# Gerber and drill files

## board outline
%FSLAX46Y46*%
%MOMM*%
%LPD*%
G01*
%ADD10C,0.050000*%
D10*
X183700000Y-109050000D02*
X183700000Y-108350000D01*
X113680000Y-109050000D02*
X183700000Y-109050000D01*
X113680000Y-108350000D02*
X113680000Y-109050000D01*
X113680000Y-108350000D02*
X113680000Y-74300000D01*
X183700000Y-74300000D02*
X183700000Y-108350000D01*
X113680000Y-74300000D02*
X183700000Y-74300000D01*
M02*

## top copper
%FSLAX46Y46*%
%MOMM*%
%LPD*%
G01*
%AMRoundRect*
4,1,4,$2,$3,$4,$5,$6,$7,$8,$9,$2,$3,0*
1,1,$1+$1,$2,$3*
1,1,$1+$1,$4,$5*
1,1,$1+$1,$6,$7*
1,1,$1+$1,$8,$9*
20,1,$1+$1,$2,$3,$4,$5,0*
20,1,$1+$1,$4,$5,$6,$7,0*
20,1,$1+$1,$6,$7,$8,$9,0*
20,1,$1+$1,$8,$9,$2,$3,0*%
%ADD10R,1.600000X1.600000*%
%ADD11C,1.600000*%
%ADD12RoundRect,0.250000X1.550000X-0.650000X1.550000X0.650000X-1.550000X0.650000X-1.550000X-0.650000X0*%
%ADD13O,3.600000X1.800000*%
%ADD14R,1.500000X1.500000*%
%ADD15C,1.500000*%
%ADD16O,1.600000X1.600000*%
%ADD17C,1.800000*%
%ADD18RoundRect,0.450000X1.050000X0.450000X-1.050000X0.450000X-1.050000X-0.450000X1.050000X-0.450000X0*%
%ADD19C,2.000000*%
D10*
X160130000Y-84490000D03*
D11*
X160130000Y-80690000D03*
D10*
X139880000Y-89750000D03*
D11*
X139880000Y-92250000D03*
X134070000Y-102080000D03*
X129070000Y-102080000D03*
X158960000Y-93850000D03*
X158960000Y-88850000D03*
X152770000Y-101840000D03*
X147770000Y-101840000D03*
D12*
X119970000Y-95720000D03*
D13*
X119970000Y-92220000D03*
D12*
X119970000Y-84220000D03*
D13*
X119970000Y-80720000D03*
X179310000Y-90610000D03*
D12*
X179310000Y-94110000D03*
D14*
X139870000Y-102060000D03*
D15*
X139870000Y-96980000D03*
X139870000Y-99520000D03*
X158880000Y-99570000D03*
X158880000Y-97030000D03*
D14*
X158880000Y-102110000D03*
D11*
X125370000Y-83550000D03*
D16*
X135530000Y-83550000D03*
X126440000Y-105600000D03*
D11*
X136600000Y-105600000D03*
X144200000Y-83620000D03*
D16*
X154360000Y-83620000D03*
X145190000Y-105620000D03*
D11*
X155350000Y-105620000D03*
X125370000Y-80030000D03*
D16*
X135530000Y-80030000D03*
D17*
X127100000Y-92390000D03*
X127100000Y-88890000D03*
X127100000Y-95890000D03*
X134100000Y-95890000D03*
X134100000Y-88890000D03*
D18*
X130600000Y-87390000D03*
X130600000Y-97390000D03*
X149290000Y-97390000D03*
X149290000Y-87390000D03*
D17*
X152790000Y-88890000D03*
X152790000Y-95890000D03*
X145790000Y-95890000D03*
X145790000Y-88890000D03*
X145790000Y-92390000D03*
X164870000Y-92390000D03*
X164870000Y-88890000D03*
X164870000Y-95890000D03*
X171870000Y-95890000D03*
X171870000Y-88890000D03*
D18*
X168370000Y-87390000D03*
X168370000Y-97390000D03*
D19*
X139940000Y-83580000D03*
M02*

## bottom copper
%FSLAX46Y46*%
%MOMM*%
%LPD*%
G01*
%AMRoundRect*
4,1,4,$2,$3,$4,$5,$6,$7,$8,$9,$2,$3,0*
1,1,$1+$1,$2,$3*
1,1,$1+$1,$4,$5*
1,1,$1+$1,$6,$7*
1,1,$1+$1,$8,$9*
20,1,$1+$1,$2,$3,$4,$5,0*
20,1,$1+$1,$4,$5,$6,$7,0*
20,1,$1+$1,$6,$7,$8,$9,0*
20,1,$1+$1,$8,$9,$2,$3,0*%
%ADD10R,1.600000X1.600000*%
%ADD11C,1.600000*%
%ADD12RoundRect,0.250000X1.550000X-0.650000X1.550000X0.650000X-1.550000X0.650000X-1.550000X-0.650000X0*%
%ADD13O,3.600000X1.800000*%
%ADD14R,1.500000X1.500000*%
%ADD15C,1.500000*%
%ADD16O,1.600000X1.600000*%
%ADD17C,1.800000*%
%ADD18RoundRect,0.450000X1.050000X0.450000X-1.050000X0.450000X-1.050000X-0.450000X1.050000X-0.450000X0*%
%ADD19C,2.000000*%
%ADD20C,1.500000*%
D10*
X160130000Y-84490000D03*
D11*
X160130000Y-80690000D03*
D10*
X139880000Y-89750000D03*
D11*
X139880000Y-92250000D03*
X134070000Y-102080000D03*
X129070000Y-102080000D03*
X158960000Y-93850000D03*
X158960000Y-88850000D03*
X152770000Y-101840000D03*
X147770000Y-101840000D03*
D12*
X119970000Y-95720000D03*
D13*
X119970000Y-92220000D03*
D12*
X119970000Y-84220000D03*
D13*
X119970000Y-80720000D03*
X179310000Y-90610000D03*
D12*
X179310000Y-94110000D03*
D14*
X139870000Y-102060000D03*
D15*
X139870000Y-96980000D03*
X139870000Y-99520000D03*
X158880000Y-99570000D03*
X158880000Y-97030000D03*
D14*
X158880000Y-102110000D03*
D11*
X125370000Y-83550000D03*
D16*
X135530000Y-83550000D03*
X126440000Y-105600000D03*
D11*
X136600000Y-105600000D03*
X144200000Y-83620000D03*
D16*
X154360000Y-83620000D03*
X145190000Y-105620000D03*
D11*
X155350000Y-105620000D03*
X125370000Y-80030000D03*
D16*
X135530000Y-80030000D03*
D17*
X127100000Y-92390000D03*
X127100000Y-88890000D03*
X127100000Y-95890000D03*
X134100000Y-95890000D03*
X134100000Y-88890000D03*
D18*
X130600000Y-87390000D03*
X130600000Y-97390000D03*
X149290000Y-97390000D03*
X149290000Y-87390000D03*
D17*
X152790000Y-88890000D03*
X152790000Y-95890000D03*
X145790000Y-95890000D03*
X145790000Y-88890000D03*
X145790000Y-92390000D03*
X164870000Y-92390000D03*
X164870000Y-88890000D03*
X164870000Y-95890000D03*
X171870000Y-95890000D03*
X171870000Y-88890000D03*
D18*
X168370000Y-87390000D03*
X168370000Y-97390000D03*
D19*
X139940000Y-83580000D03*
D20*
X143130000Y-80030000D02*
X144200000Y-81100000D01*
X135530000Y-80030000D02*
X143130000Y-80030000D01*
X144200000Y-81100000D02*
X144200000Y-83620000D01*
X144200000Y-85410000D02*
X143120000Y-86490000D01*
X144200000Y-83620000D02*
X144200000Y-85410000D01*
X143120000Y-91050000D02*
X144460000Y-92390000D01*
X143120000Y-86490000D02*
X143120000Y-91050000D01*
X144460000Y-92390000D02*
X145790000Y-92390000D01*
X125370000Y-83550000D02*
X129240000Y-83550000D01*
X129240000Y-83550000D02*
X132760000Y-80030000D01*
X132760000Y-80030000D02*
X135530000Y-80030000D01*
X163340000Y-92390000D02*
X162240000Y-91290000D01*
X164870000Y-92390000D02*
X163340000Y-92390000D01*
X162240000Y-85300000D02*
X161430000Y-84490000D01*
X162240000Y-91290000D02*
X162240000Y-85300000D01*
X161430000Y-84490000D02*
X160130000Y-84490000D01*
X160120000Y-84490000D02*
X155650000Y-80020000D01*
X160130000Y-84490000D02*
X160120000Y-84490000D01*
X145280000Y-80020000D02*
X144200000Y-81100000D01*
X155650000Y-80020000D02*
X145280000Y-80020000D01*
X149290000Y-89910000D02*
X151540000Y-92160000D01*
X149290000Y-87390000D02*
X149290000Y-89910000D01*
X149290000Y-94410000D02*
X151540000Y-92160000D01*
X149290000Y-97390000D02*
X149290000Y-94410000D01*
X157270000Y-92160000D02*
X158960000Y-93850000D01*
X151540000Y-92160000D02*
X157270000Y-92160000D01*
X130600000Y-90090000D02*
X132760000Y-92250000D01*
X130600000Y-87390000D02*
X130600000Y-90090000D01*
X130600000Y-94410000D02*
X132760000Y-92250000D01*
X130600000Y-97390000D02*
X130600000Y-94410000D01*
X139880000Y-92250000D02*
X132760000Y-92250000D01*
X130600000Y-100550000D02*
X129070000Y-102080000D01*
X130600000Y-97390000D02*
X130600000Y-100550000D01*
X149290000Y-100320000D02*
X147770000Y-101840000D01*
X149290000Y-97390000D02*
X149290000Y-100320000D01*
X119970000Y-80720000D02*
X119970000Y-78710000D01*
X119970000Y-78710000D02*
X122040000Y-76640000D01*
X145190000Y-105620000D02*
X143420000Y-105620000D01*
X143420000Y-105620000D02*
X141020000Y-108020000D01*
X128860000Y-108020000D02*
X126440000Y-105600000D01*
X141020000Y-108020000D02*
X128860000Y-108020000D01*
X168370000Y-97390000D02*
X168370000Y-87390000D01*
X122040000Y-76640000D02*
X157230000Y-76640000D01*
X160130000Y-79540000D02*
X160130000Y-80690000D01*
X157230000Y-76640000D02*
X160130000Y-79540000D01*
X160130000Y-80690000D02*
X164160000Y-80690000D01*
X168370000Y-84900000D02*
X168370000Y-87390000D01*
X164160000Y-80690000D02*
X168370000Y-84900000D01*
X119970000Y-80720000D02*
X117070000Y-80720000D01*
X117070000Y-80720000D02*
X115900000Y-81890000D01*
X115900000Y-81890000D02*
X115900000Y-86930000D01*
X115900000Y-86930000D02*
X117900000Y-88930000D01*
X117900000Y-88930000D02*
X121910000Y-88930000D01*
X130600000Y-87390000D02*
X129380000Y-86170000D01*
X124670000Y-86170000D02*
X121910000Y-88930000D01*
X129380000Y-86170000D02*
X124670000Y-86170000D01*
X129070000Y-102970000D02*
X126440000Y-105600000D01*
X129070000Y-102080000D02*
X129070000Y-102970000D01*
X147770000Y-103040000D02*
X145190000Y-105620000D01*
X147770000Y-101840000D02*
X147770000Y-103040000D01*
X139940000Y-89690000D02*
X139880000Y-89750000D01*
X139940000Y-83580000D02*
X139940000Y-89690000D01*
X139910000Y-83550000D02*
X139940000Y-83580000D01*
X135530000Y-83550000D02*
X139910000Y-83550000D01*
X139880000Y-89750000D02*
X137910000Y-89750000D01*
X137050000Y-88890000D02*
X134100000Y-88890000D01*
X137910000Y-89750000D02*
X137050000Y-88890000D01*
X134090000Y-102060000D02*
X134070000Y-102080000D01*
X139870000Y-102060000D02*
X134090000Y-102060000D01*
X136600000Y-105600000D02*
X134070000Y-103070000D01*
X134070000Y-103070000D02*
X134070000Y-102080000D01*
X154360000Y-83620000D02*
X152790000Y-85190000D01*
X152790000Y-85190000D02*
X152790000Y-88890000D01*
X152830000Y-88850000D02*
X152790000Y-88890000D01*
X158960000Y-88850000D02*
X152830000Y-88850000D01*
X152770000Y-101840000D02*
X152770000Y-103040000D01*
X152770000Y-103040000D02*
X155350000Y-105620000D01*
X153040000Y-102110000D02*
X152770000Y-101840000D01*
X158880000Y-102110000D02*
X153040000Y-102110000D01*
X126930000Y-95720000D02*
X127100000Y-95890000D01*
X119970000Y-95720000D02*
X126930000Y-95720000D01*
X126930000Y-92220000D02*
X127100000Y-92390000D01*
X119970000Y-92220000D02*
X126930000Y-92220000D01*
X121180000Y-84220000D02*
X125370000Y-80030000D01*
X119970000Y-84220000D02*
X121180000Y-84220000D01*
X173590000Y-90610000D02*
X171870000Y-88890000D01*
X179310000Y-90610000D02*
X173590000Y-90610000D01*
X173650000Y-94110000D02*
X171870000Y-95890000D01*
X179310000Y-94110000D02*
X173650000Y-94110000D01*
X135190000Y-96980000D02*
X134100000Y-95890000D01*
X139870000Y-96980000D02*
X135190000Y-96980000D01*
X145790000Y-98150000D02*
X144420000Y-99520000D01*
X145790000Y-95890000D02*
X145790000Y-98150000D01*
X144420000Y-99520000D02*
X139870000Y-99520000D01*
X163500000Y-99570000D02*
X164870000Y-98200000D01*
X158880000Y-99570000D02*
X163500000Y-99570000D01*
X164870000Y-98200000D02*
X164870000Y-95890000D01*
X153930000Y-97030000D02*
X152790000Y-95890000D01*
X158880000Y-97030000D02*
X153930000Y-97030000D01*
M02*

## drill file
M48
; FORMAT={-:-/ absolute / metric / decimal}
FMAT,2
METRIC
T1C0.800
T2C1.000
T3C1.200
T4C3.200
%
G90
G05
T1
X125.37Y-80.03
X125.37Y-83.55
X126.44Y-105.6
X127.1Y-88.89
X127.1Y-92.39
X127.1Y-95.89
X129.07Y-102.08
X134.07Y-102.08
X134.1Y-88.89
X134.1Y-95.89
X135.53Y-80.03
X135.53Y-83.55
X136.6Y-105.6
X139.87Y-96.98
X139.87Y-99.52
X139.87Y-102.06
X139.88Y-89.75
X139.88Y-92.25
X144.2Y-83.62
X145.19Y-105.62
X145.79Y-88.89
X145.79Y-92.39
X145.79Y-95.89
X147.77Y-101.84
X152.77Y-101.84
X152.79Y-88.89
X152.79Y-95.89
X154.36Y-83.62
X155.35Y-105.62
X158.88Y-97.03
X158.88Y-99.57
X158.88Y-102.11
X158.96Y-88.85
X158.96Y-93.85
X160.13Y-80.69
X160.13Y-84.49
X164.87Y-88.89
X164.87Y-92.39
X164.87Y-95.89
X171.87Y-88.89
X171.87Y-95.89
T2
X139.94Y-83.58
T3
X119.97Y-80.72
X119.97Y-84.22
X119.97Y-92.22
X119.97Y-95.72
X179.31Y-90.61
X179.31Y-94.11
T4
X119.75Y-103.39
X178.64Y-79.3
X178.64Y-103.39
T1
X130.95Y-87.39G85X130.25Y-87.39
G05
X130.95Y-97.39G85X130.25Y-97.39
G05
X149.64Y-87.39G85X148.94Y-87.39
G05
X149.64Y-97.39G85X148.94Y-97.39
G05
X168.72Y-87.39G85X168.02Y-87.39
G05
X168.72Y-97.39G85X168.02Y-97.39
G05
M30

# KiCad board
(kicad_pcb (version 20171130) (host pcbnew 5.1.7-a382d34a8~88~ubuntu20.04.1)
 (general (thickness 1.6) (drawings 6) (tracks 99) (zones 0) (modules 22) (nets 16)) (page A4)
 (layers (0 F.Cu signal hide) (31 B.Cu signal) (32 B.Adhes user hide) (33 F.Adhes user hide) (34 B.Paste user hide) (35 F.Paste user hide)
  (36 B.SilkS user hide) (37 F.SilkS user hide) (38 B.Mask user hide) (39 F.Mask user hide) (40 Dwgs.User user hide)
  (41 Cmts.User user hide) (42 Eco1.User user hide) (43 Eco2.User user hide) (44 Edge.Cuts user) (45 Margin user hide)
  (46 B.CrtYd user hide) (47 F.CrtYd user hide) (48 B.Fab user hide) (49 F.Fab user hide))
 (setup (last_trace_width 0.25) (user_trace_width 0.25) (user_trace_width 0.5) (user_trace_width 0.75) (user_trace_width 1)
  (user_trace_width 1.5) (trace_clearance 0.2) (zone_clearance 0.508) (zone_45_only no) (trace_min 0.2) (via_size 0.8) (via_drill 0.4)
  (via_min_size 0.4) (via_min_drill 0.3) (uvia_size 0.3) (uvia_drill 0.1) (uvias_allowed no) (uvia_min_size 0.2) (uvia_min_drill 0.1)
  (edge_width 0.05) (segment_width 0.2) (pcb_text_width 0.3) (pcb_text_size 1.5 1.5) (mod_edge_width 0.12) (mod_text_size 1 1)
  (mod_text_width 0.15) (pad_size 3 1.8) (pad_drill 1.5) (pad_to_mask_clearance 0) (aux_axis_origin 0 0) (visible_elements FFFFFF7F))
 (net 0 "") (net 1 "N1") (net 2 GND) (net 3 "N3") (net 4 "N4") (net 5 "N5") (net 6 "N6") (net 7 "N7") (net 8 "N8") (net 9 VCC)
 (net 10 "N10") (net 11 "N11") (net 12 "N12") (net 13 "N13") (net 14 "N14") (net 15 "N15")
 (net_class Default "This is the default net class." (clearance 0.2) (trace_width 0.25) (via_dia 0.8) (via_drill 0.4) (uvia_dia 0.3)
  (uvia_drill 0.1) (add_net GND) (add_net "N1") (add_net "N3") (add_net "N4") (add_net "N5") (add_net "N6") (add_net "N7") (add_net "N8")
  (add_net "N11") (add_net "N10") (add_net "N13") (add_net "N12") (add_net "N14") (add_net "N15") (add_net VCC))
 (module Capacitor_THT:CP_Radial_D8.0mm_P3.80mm (layer F.Cu) (at 160.13 84.49 90)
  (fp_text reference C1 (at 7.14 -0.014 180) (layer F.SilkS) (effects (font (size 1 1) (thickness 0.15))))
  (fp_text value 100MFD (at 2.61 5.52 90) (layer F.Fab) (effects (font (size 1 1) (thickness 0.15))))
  (pad 1 thru_hole rect (at 0 0 90) (size 1.6 1.6) (drill 0.8) (layers *.Cu *.Mask) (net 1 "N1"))
  (pad 2 thru_hole circle (at 3.8 0 90) (size 1.6 1.6) (drill 0.8) (layers *.Cu *.Mask) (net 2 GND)))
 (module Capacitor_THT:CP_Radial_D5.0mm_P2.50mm (layer F.Cu) (at 139.88 89.75 270)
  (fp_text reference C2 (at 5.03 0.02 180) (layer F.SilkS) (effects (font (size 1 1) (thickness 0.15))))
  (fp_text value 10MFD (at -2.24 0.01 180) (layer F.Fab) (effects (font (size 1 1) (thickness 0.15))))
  (pad 1 thru_hole rect (at 0 0 270) (size 1.6 1.6) (drill 0.8) (layers *.Cu *.Mask) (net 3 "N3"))
  (pad 2 thru_hole circle (at 2.5 0 270) (size 1.6 1.6) (drill 0.8) (layers *.Cu *.Mask) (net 2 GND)))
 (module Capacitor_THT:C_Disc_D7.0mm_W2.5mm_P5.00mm (layer F.Cu) (at 134.07 102.08 180)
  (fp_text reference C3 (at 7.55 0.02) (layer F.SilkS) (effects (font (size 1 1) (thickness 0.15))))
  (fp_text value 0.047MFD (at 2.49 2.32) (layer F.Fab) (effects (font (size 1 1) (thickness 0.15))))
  (pad 1 thru_hole circle (at 0 0 180) (size 1.6 1.6) (drill 0.8) (layers *.Cu *.Mask) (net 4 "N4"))
  (pad 2 thru_hole circle (at 5 0 180) (size 1.6 1.6) (drill 0.8) (layers *.Cu *.Mask) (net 2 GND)))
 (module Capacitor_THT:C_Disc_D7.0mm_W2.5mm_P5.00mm (layer F.Cu) (at 158.96 88.85 270)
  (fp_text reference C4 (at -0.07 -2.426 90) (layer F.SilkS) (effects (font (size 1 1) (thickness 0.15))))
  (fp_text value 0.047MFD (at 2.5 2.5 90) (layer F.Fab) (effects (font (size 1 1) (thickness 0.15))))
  (pad 2 thru_hole circle (at 5 0 270) (size 1.6 1.6) (drill 0.8) (layers *.Cu *.Mask) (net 2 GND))
  (pad 1 thru_hole circle (at 0 0 270) (size 1.6 1.6) (drill 0.8) (layers *.Cu *.Mask) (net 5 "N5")))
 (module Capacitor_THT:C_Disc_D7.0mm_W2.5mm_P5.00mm (layer F.Cu) (at 152.77 101.84 180)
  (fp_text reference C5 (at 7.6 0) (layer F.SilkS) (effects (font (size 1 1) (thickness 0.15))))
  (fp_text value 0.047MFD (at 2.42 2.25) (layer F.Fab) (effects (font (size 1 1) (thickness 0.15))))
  (pad 1 thru_hole circle (at 0 0 180) (size 1.6 1.6) (drill 0.8) (layers *.Cu *.Mask) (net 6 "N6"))
  (pad 2 thru_hole circle (at 5 0 180) (size 1.6 1.6) (drill 0.8) (layers *.Cu *.Mask) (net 2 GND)))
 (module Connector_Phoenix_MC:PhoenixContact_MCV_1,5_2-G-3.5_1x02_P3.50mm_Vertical (layer F.Cu) (at 119.97 95.72 90)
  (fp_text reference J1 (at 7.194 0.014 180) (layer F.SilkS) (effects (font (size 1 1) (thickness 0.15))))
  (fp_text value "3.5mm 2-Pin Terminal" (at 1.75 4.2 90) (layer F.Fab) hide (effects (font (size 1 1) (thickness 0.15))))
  (pad 1 thru_hole roundrect (at 0 0 90) (size 1.8 3.6) (drill 1.2) (layers *.Cu *.Mask) (roundrect_rratio 0.138889) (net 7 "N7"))
  (pad 2 thru_hole oval (at 3.5 0 90) (size 1.8 3.6) (drill 1.2) (layers *.Cu *.Mask) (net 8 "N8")))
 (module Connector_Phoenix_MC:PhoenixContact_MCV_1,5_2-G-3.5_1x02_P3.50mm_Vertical (layer F.Cu) (at 119.97 84.22 90)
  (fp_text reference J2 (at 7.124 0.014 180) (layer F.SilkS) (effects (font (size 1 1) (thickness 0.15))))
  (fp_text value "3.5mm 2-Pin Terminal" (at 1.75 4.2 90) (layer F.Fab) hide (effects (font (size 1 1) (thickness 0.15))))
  (pad 1 thru_hole roundrect (at 0 0 90) (size 1.8 3.6) (drill 1.2) (layers *.Cu *.Mask) (roundrect_rratio 0.138889) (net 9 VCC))
  (pad 2 thru_hole oval (at 3.5 0 90) (size 1.8 3.6) (drill 1.2) (layers *.Cu *.Mask) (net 2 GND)))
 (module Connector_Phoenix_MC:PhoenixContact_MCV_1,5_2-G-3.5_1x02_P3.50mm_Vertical (layer F.Cu) (at 179.31 94.11 90)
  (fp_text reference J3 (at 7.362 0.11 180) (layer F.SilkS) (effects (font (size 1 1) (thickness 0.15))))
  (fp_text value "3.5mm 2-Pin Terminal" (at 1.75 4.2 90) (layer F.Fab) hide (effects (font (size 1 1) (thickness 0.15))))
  (pad 2 thru_hole oval (at 3.5 0 90) (size 1.8 3.6) (drill 1.2) (layers *.Cu *.Mask) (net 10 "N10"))
  (pad 1 thru_hole roundrect (at 0 0 90) (size 1.8 3.6) (drill 1.2) (layers *.Cu *.Mask) (roundrect_rratio 0.138889) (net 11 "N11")))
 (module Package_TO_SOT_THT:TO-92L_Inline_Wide (layer F.Cu) (at 139.87 102.06 90)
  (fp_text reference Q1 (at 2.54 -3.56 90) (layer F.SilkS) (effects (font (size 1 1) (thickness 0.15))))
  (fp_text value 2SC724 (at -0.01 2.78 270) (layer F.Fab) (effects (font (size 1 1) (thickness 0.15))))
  (pad 1 thru_hole rect (at 0 0 90) (size 1.5 1.5) (drill 0.8) (layers *.Cu *.Mask) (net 4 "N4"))
  (pad 3 thru_hole circle (at 5.08 0 90) (size 1.5 1.5) (drill 0.8) (layers *.Cu *.Mask) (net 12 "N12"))
  (pad 2 thru_hole circle (at 2.54 0 90) (size 1.5 1.5) (drill 0.8) (layers *.Cu *.Mask) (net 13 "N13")))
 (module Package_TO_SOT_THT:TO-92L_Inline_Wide (layer F.Cu) (at 158.88 102.11 90)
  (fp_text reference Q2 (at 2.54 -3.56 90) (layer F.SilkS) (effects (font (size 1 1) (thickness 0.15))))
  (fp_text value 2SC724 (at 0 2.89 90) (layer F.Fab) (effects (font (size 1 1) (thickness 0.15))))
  (pad 2 thru_hole circle (at 2.54 0 90) (size 1.5 1.5) (drill 0.8) (layers *.Cu *.Mask) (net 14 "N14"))
  (pad 3 thru_hole circle (at 5.08 0 90) (size 1.5 1.5) (drill 0.8) (layers *.Cu *.Mask) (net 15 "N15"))
  (pad 1 thru_hole rect (at 0 0 90) (size 1.5 1.5) (drill 0.8) (layers *.Cu *.Mask) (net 6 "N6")))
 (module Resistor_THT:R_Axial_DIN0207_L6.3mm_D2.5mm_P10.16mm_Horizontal (layer F.Cu) (at 125.37 83.55)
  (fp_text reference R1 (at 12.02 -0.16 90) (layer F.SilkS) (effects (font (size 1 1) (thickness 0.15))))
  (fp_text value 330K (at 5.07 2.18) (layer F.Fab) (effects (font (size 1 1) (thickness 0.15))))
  (pad 1 thru_hole circle (at 0 0) (size 1.6 1.6) (drill 0.8) (layers *.Cu *.Mask) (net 1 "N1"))
  (pad 2 thru_hole oval (at 10.16 0) (size 1.6 1.6) (drill 0.8) (layers *.Cu *.Mask) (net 3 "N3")))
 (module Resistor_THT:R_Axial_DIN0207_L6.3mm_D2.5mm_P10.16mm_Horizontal (layer F.Cu) (at 136.6 105.6 180)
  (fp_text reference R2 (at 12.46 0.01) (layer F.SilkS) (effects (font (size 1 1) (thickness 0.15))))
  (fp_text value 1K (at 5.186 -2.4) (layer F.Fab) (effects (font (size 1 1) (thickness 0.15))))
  (pad 2 thru_hole oval (at 10.16 0 180) (size 1.6 1.6) (drill 0.8) (layers *.Cu *.Mask) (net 2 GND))
  (pad 1 thru_hole circle (at 0 0 180) (size 1.6 1.6) (drill 0.8) (layers *.Cu *.Mask) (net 4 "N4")))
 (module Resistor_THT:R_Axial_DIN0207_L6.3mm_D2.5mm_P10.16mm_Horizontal (layer F.Cu) (at 144.2 83.62)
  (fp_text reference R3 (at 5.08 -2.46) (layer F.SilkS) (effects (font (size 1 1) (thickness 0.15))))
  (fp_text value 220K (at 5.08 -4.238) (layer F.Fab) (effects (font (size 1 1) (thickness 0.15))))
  (pad 1 thru_hole circle (at 0 0) (size 1.6 1.6) (drill 0.8) (layers *.Cu *.Mask) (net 1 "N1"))
  (pad 2 thru_hole oval (at 10.16 0) (size 1.6 1.6) (drill 0.8) (layers *.Cu *.Mask) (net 5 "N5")))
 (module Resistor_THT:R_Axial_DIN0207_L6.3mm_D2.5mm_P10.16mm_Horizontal (layer F.Cu) (at 155.35 105.62 180)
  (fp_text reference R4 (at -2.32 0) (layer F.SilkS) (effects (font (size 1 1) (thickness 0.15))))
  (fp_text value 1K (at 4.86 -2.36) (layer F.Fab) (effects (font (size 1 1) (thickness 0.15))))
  (pad 2 thru_hole oval (at 10.16 0 180) (size 1.6 1.6) (drill 0.8) (layers *.Cu *.Mask) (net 2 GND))
  (pad 1 thru_hole circle (at 0 0 180) (size 1.6 1.6) (drill 0.8) (layers *.Cu *.Mask) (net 6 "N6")))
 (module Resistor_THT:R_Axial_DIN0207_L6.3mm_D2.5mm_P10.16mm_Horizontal (layer F.Cu) (at 125.37 80.03)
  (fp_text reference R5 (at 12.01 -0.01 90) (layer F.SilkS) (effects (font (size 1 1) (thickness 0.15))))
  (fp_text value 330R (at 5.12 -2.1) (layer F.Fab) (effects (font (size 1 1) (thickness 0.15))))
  (pad 1 thru_hole circle (at 0 0) (size 1.6 1.6) (drill 0.8) (layers *.Cu *.Mask) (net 9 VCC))
  (pad 2 thru_hole oval (at 10.16 0) (size 1.6 1.6) (drill 0.8) (layers *.Cu *.Mask) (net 1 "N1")))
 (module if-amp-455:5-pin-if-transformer (layer F.Cu) (at 127.1 92.39 90)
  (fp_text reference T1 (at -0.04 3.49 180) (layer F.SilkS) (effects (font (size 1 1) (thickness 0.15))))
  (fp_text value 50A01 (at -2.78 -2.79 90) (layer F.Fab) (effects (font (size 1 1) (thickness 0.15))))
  (pad 2 thru_hole circle (at 0 0 90) (size 1.8 1.8) (drill 0.8) (layers *.Cu *.Mask) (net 8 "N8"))
  (pad 1 thru_hole circle (at 3.5 0 90) (size 1.8 1.8) (drill 0.8) (layers *.Cu *.Mask))
  (pad 3 thru_hole circle (at -3.5 0 90) (size 1.8 1.8) (drill 0.8) (layers *.Cu *.Mask) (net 7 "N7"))
  (pad 4 thru_hole circle (at -3.5 7 90) (size 1.8 1.8) (drill 0.8) (layers *.Cu *.Mask) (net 12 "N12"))
  (pad 5 thru_hole circle (at 3.5 7 90) (size 1.8 1.8) (drill 0.8) (layers *.Cu *.Mask) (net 3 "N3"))
  (pad 6 thru_hole roundrect (at 5 3.5 180) (size 3 1.8) (drill oval 1.5 0.8) (layers *.Cu *.Mask) (roundrect_rratio 0.25) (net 2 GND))
  (pad 6 thru_hole roundrect (at -5 3.5 180) (size 3 1.8) (drill oval 1.5 0.8) (layers *.Cu *.Mask) (roundrect_rratio 0.25) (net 2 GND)))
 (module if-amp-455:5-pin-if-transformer (layer F.Cu) (at 145.79 92.39 90)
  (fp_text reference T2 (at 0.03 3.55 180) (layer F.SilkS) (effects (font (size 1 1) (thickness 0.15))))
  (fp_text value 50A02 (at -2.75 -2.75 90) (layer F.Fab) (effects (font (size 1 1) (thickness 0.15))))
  (pad 6 thru_hole roundrect (at -5 3.5 180) (size 3 1.8) (drill oval 1.5 0.8) (layers *.Cu *.Mask) (roundrect_rratio 0.25) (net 2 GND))
  (pad 6 thru_hole roundrect (at 5 3.5 180) (size 3 1.8) (drill oval 1.5 0.8) (layers *.Cu *.Mask) (roundrect_rratio 0.25) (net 2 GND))
  (pad 5 thru_hole circle (at 3.5 7 90) (size 1.8 1.8) (drill 0.8) (layers *.Cu *.Mask) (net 5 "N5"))
  (pad 4 thru_hole circle (at -3.5 7 90) (size 1.8 1.8) (drill 0.8) (layers *.Cu *.Mask) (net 15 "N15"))
  (pad 3 thru_hole circle (at -3.5 0 90) (size 1.8 1.8) (drill 0.8) (layers *.Cu *.Mask) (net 13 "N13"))
  (pad 1 thru_hole circle (at 3.5 0 90) (size 1.8 1.8) (drill 0.8) (layers *.Cu *.Mask))
  (pad 2 thru_hole circle (at 0 0 90) (size 1.8 1.8) (drill 0.8) (layers *.Cu *.Mask) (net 1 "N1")))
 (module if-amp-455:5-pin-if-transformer (layer F.Cu) (at 164.87 92.39 90)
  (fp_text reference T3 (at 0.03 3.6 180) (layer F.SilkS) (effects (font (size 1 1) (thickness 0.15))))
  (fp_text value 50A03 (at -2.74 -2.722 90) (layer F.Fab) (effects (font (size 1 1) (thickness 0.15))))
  (pad 2 thru_hole circle (at 0 0 90) (size 1.8 1.8) (drill 0.8) (layers *.Cu *.Mask) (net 1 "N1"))
  (pad 1 thru_hole circle (at 3.5 0 90) (size 1.8 1.8) (drill 0.8) (layers *.Cu *.Mask))
  (pad 3 thru_hole circle (at -3.5 0 90) (size 1.8 1.8) (drill 0.8) (layers *.Cu *.Mask) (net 14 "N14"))
  (pad 4 thru_hole circle (at -3.5 7 90) (size 1.8 1.8) (drill 0.8) (layers *.Cu *.Mask) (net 11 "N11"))
  (pad 5 thru_hole circle (at 3.5 7 90) (size 1.8 1.8) (drill 0.8) (layers *.Cu *.Mask) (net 10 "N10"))
  (pad 6 thru_hole roundrect (at 5 3.5 180) (size 3 1.8) (drill oval 1.5 0.8) (layers *.Cu *.Mask) (roundrect_rratio 0.25) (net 2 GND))
  (pad 6 thru_hole roundrect (at -5 3.5 180) (size 3 1.8) (drill oval 1.5 0.8) (layers *.Cu *.Mask) (roundrect_rratio 0.25) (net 2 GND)))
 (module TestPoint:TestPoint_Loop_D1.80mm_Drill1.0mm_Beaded (layer F.Cu) (at 139.94 83.58)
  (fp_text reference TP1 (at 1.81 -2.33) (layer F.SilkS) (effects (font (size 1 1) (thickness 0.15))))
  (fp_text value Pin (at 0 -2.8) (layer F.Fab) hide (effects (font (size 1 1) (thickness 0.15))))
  (pad 1 thru_hole circle (at 0 0) (size 2 2) (drill 1) (layers *.Cu *.Mask) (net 3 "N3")))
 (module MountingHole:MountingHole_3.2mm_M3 (layer F.Cu) (at 119.75 103.39)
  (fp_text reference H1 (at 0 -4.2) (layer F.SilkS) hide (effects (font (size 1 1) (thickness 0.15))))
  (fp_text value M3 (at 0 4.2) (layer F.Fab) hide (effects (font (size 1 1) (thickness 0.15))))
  (pad 1 np_thru_hole circle (at 0 0) (size 3.2 3.2) (drill 3.2) (layers *.Cu *.Mask)))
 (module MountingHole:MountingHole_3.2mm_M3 (layer F.Cu) (at 178.64 103.39)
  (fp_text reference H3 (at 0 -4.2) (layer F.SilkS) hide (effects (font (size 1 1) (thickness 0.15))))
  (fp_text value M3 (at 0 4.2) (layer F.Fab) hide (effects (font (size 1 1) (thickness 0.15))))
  (pad 1 np_thru_hole circle (at 0 0) (size 3.2 3.2) (drill 3.2) (layers *.Cu *.Mask)))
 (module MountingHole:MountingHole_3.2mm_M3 (layer F.Cu) (at 178.64 79.3)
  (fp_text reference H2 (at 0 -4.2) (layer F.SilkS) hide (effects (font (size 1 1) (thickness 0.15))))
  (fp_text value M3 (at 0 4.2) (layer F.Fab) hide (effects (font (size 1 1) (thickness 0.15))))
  (pad 1 np_thru_hole circle (at 0 0) (size 3.2 3.2) (drill 3.2) (layers *.Cu *.Mask)))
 (gr_line (start 183.7 109.05) (end 183.7 108.35) (layer Edge.Cuts) (width 0.05))
 (gr_line (start 113.68 109.05) (end 183.7 109.05) (layer Edge.Cuts) (width 0.05))
 (gr_line (start 113.68 108.35) (end 113.68 109.05) (layer Edge.Cuts) (width 0.05))
 (gr_line (start 113.68 108.35) (end 113.68 74.3) (layer Edge.Cuts) (width 0.05))
 (gr_line (start 183.7 74.3) (end 183.7 108.35) (layer Edge.Cuts) (width 0.05))
 (gr_line (start 113.68 74.3) (end 183.7 74.3) (layer Edge.Cuts) (width 0.05))
 (segment (start 143.13 80.03) (end 144.2 81.1) (width 1.5) (layer B.Cu) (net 1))
 (segment (start 135.53 80.03) (end 143.13 80.03) (width 1.5) (layer B.Cu) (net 1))
 (segment (start 144.2 81.1) (end 144.2 83.62) (width 1.5) (layer B.Cu) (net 1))
 (segment (start 144.2 85.41) (end 143.12 86.49) (width 1.5) (layer B.Cu) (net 1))
 (segment (start 144.2 83.62) (end 144.2 85.41) (width 1.5) (layer B.Cu) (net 1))
 (segment (start 143.12 91.05) (end 144.46 92.39) (width 1.5) (layer B.Cu) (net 1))
 (segment (start 143.12 86.49) (end 143.12 91.05) (width 1.5) (layer B.Cu) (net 1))
 (segment (start 144.46 92.39) (end 145.79 92.39) (width 1.5) (layer B.Cu) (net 1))
 (segment (start 125.37 83.55) (end 129.24 83.55) (width 1.5) (layer B.Cu) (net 1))
 (segment (start 129.24 83.55) (end 132.76 80.03) (width 1.5) (layer B.Cu) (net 1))
 (segment (start 132.76 80.03) (end 135.53 80.03) (width 1.5) (layer B.Cu) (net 1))
 (segment (start 163.34 92.39) (end 162.24 91.29) (width 1.5) (layer B.Cu) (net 1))
 (segment (start 164.87 92.39) (end 163.34 92.39) (width 1.5) (layer B.Cu) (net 1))
 (segment (start 162.24 85.3) (end 161.43 84.49) (width 1.5) (layer B.Cu) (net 1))
 (segment (start 162.24 91.29) (end 162.24 85.3) (width 1.5) (layer B.Cu) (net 1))
 (segment (start 161.43 84.49) (end 160.13 84.49) (width 1.5) (layer B.Cu) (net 1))
 (segment (start 160.12 84.49) (end 155.65 80.02) (width 1.5) (layer B.Cu) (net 1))
 (segment (start 160.13 84.49) (end 160.12 84.49) (width 1.5) (layer B.Cu) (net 1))
 (segment (start 145.28 80.02) (end 144.2 81.1) (width 1.5) (layer B.Cu) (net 1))
 (segment (start 155.65 80.02) (end 145.28 80.02) (width 1.5) (layer B.Cu) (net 1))
 (segment (start 149.29 89.91) (end 151.54 92.16) (width 1.5) (layer B.Cu) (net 2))
 (segment (start 149.29 87.39) (end 149.29 89.91) (width 1.5) (layer B.Cu) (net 2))
 (segment (start 149.29 94.41) (end 151.54 92.16) (width 1.5) (layer B.Cu) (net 2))
 (segment (start 149.29 97.39) (end 149.29 94.41) (width 1.5) (layer B.Cu) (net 2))
 (segment (start 157.27 92.16) (end 158.96 93.85) (width 1.5) (layer B.Cu) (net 2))
 (segment (start 151.54 92.16) (end 157.27 92.16) (width 1.5) (layer B.Cu) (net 2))
 (segment (start 130.6 90.09) (end 132.76 92.25) (width 1.5) (layer B.Cu) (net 2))
 (segment (start 130.6 87.39) (end 130.6 90.09) (width 1.5) (layer B.Cu) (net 2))
 (segment (start 130.6 94.41) (end 132.76 92.25) (width 1.5) (layer B.Cu) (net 2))
 (segment (start 130.6 97.39) (end 130.6 94.41) (width 1.5) (layer B.Cu) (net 2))
 (segment (start 139.88 92.25) (end 132.76 92.25) (width 1.5) (layer B.Cu) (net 2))
 (segment (start 130.6 100.55) (end 129.07 102.08) (width 1.5) (layer B.Cu) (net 2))
 (segment (start 130.6 97.39) (end 130.6 100.55) (width 1.5) (layer B.Cu) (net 2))
 (segment (start 149.29 100.32) (end 147.77 101.84) (width 1.5) (layer B.Cu) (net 2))
 (segment (start 149.29 97.39) (end 149.29 100.32) (width 1.5) (layer B.Cu) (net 2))
 (segment (start 119.97 80.72) (end 119.97 78.71) (width 1.5) (layer B.Cu) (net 2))
 (segment (start 119.97 78.71) (end 122.04 76.64) (width 1.5) (layer B.Cu) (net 2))
 (segment (start 145.19 105.62) (end 143.42 105.62) (width 1.5) (layer B.Cu) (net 2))
 (segment (start 143.42 105.62) (end 141.02 108.02) (width 1.5) (layer B.Cu) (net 2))
 (segment (start 128.86 108.02) (end 126.44 105.6) (width 1.5) (layer B.Cu) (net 2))
 (segment (start 141.02 108.02) (end 128.86 108.02) (width 1.5) (layer B.Cu) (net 2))
 (segment (start 168.37 97.39) (end 168.37 87.39) (width 1.5) (layer B.Cu) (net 2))
 (segment (start 122.04 76.64) (end 157.23 76.64) (width 1.5) (layer B.Cu) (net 2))
 (segment (start 160.13 79.54) (end 160.13 80.69) (width 1.5) (layer B.Cu) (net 2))
 (segment (start 157.23 76.64) (end 160.13 79.54) (width 1.5) (layer B.Cu) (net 2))
 (segment (start 160.13 80.69) (end 164.16 80.69) (width 1.5) (layer B.Cu) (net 2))
 (segment (start 168.37 84.9) (end 168.37 87.39) (width 1.5) (layer B.Cu) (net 2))
 (segment (start 164.16 80.69) (end 168.37 84.9) (width 1.5) (layer B.Cu) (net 2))
 (segment (start 119.97 80.72) (end 117.07 80.72) (width 1.5) (layer B.Cu) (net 2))
 (segment (start 117.07 80.72) (end 115.9 81.89) (width 1.5) (layer B.Cu) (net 2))
 (segment (start 115.9 81.89) (end 115.9 86.93) (width 1.5) (layer B.Cu) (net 2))
 (segment (start 115.9 86.93) (end 117.9 88.93) (width 1.5) (layer B.Cu) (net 2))
 (segment (start 117.9 88.93) (end 121.91 88.93) (width 1.5) (layer B.Cu) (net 2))
 (segment (start 130.6 87.39) (end 129.38 86.17) (width 1.5) (layer B.Cu) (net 2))
 (segment (start 124.67 86.17) (end 121.91 88.93) (width 1.5) (layer B.Cu) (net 2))
 (segment (start 129.38 86.17) (end 124.67 86.17) (width 1.5) (layer B.Cu) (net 2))
 (segment (start 129.07 102.97) (end 126.44 105.6) (width 1.5) (layer B.Cu) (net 2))
 (segment (start 129.07 102.08) (end 129.07 102.97) (width 1.5) (layer B.Cu) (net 2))
 (segment (start 147.77 103.04) (end 145.19 105.62) (width 1.5) (layer B.Cu) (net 2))
 (segment (start 147.77 101.84) (end 147.77 103.04) (width 1.5) (layer B.Cu) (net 2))
 (segment (start 139.94 89.69) (end 139.88 89.75) (width 1.5) (layer B.Cu) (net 3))
 (segment (start 139.94 83.58) (end 139.94 89.69) (width 1.5) (layer B.Cu) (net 3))
 (segment (start 139.91 83.55) (end 139.94 83.58) (width 1.5) (layer B.Cu) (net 3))
 (segment (start 135.53 83.55) (end 139.91 83.55) (width 1.5) (layer B.Cu) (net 3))
 (segment (start 139.88 89.75) (end 137.91 89.75) (width 1.5) (layer B.Cu) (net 3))
 (segment (start 137.05 88.89) (end 134.1 88.89) (width 1.5) (layer B.Cu) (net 3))
 (segment (start 137.91 89.75) (end 137.05 88.89) (width 1.5) (layer B.Cu) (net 3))
 (segment (start 134.09 102.06) (end 134.07 102.08) (width 1.5) (layer B.Cu) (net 4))
 (segment (start 139.87 102.06) (end 134.09 102.06) (width 1.5) (layer B.Cu) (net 4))
 (segment (start 136.6 105.6) (end 134.07 103.07) (width 1.5) (layer B.Cu) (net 4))
 (segment (start 134.07 103.07) (end 134.07 102.08) (width 1.5) (layer B.Cu) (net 4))
 (segment (start 154.36 83.62) (end 152.79 85.19) (width 1.5) (layer B.Cu) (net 5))
 (segment (start 152.79 85.19) (end 152.79 88.89) (width 1.5) (layer B.Cu) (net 5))
 (segment (start 152.83 88.85) (end 152.79 88.89) (width 1.5) (layer B.Cu) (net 5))
 (segment (start 158.96 88.85) (end 152.83 88.85) (width 1.5) (layer B.Cu) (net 5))
 (segment (start 152.77 101.84) (end 152.77 103.04) (width 1.5) (layer B.Cu) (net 6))
 (segment (start 152.77 103.04) (end 155.35 105.62) (width 1.5) (layer B.Cu) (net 6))
 (segment (start 153.04 102.11) (end 152.77 101.84) (width 1.5) (layer B.Cu) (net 6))
 (segment (start 158.88 102.11) (end 153.04 102.11) (width 1.5) (layer B.Cu) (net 6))
 (segment (start 126.93 95.72) (end 127.1 95.89) (width 1.5) (layer B.Cu) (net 7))
 (segment (start 119.97 95.72) (end 126.93 95.72) (width 1.5) (layer B.Cu) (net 7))
 (segment (start 126.93 92.22) (end 127.1 92.39) (width 1.5) (layer B.Cu) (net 8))
 (segment (start 119.97 92.22) (end 126.93 92.22) (width 1.5) (layer B.Cu) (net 8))
 (segment (start 121.18 84.22) (end 125.37 80.03) (width 1.5) (layer B.Cu) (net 9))
 (segment (start 119.97 84.22) (end 121.18 84.22) (width 1.5) (layer B.Cu) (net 9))
 (segment (start 173.59 90.61) (end 171.87 88.89) (width 1.5) (layer B.Cu) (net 10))
 (segment (start 179.31 90.61) (end 173.59 90.61) (width 1.5) (layer B.Cu) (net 10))
 (segment (start 173.65 94.11) (end 171.87 95.89) (width 1.5) (layer B.Cu) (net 11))
 (segment (start 179.31 94.11) (end 173.65 94.11) (width 1.5) (layer B.Cu) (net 11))
 (segment (start 135.19 96.98) (end 134.1 95.89) (width 1.5) (layer B.Cu) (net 12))
 (segment (start 139.87 96.98) (end 135.19 96.98) (width 1.5) (layer B.Cu) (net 12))
 (segment (start 145.79 98.15) (end 144.42 99.52) (width 1.5) (layer B.Cu) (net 13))
 (segment (start 145.79 95.89) (end 145.79 98.15) (width 1.5) (layer B.Cu) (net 13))
 (segment (start 144.42 99.52) (end 139.87 99.52) (width 1.5) (layer B.Cu) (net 13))
 (segment (start 163.5 99.57) (end 164.87 98.2) (width 1.5) (layer B.Cu) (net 14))
 (segment (start 158.88 99.57) (end 163.5 99.57) (width 1.5) (layer B.Cu) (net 14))
 (segment (start 164.87 98.2) (end 164.87 95.89) (width 1.5) (layer B.Cu) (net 14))
 (segment (start 153.93 97.03) (end 152.79 95.89) (width 1.5) (layer B.Cu) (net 15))
 (segment (start 158.88 97.03) (end 153.93 97.03) (width 1.5) (layer B.Cu) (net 15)))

